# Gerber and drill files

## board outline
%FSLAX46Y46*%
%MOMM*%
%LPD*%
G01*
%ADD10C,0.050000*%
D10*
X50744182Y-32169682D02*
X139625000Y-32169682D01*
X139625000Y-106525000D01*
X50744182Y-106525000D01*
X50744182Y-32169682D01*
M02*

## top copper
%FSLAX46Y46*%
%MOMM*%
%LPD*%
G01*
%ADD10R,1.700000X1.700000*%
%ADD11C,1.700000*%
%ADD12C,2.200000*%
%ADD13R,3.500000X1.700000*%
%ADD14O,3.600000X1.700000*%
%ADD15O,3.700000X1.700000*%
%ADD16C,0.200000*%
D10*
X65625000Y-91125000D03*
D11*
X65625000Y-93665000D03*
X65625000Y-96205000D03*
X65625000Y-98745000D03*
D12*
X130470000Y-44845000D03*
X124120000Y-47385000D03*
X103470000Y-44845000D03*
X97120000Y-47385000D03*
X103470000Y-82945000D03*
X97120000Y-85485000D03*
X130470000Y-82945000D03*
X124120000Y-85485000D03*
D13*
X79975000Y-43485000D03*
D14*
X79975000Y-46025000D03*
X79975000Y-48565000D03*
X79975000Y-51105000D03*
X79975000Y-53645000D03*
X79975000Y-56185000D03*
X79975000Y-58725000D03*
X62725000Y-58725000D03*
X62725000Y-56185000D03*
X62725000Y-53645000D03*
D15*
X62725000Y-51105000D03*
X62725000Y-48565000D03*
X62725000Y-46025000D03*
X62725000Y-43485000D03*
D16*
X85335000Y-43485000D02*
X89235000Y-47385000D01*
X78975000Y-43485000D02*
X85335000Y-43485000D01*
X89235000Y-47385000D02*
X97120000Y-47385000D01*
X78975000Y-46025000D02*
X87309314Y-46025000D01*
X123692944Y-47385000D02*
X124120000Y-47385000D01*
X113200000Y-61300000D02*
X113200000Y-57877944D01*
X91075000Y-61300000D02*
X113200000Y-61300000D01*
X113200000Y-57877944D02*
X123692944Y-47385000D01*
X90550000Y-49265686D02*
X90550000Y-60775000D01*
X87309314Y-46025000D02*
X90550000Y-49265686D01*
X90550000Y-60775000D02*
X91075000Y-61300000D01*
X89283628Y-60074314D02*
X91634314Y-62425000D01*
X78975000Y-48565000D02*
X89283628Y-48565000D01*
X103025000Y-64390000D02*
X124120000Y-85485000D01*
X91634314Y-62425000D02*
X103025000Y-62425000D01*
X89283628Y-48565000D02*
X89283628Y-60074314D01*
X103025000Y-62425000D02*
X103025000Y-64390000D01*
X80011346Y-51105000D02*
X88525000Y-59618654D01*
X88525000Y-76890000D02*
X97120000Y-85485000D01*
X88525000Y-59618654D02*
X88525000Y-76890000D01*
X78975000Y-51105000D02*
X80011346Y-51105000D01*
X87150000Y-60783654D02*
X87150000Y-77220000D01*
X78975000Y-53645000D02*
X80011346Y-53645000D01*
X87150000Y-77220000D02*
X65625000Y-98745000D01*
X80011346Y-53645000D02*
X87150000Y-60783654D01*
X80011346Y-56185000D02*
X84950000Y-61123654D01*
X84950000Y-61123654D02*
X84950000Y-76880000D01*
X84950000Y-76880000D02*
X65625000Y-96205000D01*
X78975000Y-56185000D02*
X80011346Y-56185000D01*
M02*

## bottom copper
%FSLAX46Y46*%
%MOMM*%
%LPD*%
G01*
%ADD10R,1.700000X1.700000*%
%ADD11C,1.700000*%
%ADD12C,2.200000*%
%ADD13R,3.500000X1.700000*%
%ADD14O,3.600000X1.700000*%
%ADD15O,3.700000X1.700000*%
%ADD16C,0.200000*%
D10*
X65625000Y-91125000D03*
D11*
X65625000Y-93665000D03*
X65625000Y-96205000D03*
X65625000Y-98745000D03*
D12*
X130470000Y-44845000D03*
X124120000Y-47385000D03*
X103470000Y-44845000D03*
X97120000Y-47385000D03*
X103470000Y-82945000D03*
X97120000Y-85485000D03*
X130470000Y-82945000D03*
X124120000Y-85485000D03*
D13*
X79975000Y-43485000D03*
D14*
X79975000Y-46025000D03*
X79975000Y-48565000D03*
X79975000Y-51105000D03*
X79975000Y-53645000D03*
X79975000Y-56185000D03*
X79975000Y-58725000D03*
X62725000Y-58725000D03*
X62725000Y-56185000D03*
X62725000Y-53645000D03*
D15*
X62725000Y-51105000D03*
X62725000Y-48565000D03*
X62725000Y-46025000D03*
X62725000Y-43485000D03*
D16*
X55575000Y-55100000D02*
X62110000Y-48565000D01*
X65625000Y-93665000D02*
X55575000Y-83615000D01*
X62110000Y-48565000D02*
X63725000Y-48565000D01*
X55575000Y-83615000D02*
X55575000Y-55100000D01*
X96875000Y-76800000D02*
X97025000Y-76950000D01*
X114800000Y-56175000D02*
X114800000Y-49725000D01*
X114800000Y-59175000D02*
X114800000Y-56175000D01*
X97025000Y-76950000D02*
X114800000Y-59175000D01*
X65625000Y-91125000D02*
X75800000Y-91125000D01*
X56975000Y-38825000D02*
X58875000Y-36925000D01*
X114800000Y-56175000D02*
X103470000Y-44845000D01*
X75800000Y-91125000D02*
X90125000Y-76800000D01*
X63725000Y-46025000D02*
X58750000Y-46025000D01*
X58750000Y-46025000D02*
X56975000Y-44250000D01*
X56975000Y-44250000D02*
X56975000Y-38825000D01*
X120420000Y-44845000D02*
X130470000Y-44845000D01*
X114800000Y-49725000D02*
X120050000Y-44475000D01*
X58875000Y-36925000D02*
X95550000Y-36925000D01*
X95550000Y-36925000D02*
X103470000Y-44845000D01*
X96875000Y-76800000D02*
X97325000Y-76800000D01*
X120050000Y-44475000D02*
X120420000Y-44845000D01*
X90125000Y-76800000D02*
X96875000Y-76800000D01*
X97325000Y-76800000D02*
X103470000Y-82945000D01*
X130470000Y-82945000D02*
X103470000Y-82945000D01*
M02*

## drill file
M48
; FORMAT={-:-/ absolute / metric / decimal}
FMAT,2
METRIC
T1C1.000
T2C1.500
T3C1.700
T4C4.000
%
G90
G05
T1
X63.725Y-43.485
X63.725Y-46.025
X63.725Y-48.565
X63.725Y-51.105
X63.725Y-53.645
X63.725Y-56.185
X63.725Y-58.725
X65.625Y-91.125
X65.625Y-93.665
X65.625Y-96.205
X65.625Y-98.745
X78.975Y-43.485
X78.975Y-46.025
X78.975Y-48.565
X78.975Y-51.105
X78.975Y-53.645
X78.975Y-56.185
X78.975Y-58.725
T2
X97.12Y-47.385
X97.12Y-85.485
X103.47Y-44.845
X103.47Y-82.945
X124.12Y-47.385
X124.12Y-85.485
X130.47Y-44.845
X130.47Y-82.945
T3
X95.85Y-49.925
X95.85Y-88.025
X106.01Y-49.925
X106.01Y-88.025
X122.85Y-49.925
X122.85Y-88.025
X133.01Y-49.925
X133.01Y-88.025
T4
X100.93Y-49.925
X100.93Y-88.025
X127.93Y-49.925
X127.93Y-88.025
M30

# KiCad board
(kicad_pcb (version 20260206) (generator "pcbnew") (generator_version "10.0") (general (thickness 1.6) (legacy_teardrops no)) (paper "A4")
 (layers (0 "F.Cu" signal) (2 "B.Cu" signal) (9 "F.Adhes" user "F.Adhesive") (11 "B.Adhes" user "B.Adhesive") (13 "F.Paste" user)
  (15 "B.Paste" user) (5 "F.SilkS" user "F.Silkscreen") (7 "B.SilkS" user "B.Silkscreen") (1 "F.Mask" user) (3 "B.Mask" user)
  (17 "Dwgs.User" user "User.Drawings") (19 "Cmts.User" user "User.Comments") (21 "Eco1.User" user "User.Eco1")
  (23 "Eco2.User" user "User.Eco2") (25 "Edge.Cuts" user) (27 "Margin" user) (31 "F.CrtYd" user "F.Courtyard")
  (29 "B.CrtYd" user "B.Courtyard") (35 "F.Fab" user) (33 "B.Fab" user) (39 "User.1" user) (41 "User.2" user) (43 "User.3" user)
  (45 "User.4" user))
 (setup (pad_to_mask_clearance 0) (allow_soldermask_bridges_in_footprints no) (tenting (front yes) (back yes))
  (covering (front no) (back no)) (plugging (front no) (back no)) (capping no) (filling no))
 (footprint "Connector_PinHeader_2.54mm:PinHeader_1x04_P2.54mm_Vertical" (layer "F.Cu") (at 65.625 91.125)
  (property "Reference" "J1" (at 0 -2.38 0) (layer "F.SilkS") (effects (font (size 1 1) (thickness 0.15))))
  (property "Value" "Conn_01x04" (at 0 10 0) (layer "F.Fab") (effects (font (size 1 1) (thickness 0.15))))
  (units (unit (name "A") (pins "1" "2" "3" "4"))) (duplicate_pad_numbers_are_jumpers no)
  (pad "1" thru_hole rect (at 0 0) (size 1.7 1.7) (drill 1) (layers "*.Cu" "*.Mask") (remove_unused_layers no) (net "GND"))
  (pad "2" thru_hole circle (at 0 2.54) (size 1.7 1.7) (drill 1) (layers "*.Cu" "*.Mask") (remove_unused_layers no) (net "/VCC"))
  (pad "3" thru_hole circle (at 0 5.08) (size 1.7 1.7) (drill 1) (layers "*.Cu" "*.Mask") (remove_unused_layers no) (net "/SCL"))
  (pad "4" thru_hole circle (at 0 7.62) (size 1.7 1.7) (drill 1) (layers "*.Cu" "*.Mask") (remove_unused_layers no) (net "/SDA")))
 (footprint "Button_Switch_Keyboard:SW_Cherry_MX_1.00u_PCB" (layer "F.Cu") (at 130.47 44.845)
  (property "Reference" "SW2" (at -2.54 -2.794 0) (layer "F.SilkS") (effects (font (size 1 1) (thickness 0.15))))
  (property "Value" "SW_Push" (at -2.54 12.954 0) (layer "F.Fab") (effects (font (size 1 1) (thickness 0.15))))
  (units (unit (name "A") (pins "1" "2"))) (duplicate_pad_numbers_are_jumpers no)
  (pad "" np_thru_hole circle (at -7.62 5.08) (size 1.7 1.7) (drill 1.7) (layers "*.Cu" "*.Mask"))
  (pad "" np_thru_hole circle (at -2.54 5.08) (size 4 4) (drill 4) (layers "*.Cu" "*.Mask"))
  (pad "" np_thru_hole circle (at 2.54 5.08) (size 1.7 1.7) (drill 1.7) (layers "*.Cu" "*.Mask"))
  (pad "1" thru_hole circle (at 0 0) (size 2.2 2.2) (drill 1.5) (layers "*.Cu" "*.Mask") (remove_unused_layers no) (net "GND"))
  (pad "2" thru_hole circle (at -6.35 2.54) (size 2.2 2.2) (drill 1.5) (layers "*.Cu" "*.Mask") (remove_unused_layers no)
   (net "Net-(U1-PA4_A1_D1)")))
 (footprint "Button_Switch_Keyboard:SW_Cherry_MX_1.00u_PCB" (layer "F.Cu") (at 103.47 44.845)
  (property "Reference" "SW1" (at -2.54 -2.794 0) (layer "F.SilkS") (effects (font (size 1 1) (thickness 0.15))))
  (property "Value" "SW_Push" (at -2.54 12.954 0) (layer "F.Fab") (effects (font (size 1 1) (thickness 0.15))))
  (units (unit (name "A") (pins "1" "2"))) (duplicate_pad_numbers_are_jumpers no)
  (pad "" np_thru_hole circle (at -7.62 5.08) (size 1.7 1.7) (drill 1.7) (layers "*.Cu" "*.Mask"))
  (pad "" np_thru_hole circle (at -2.54 5.08) (size 4 4) (drill 4) (layers "*.Cu" "*.Mask"))
  (pad "" np_thru_hole circle (at 2.54 5.08) (size 1.7 1.7) (drill 1.7) (layers "*.Cu" "*.Mask"))
  (pad "1" thru_hole circle (at 0 0) (size 2.2 2.2) (drill 1.5) (layers "*.Cu" "*.Mask") (remove_unused_layers no) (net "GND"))
  (pad "2" thru_hole circle (at -6.35 2.54) (size 2.2 2.2) (drill 1.5) (layers "*.Cu" "*.Mask") (remove_unused_layers no)
   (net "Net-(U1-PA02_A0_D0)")))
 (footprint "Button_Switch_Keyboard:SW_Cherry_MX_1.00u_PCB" (layer "F.Cu") (at 103.47 82.945)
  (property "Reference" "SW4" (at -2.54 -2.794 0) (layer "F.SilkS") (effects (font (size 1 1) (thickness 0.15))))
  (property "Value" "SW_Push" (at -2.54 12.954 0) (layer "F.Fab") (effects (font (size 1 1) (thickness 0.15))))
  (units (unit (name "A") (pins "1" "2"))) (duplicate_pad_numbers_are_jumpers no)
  (pad "" np_thru_hole circle (at -7.62 5.08) (size 1.7 1.7) (drill 1.7) (layers "*.Cu" "*.Mask"))
  (pad "" np_thru_hole circle (at -2.54 5.08) (size 4 4) (drill 4) (layers "*.Cu" "*.Mask"))
  (pad "" np_thru_hole circle (at 2.54 5.08) (size 1.7 1.7) (drill 1.7) (layers "*.Cu" "*.Mask"))
  (pad "1" thru_hole circle (at 0 0) (size 2.2 2.2) (drill 1.5) (layers "*.Cu" "*.Mask") (remove_unused_layers no) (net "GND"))
  (pad "2" thru_hole circle (at -6.35 2.54) (size 2.2 2.2) (drill 1.5) (layers "*.Cu" "*.Mask") (remove_unused_layers no)
   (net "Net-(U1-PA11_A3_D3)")))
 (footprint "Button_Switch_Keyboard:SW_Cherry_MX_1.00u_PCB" (layer "F.Cu") (at 130.47 82.945)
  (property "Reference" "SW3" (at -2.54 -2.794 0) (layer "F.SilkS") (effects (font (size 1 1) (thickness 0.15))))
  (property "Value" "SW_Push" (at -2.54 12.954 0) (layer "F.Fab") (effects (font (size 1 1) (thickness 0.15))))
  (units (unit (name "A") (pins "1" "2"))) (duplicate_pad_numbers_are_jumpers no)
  (pad "" np_thru_hole circle (at -7.62 5.08) (size 1.7 1.7) (drill 1.7) (layers "*.Cu" "*.Mask"))
  (pad "" np_thru_hole circle (at -2.54 5.08) (size 4 4) (drill 4) (layers "*.Cu" "*.Mask"))
  (pad "" np_thru_hole circle (at 2.54 5.08) (size 1.7 1.7) (drill 1.7) (layers "*.Cu" "*.Mask"))
  (pad "1" thru_hole circle (at 0 0) (size 2.2 2.2) (drill 1.5) (layers "*.Cu" "*.Mask") (remove_unused_layers no) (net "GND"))
  (pad "2" thru_hole circle (at -6.35 2.54) (size 2.2 2.2) (drill 1.5) (layers "*.Cu" "*.Mask") (remove_unused_layers no)
   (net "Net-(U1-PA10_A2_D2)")))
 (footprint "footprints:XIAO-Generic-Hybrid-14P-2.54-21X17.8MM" (layer "B.Cu") (at 71.35 51.105 180)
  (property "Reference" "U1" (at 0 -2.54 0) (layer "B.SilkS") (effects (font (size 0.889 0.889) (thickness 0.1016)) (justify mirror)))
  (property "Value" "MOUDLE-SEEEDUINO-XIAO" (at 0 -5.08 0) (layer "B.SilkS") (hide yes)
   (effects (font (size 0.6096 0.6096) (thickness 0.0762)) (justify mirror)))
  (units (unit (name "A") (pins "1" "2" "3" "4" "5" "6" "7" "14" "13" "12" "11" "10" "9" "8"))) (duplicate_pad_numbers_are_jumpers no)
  (pad "1" thru_hole rect (at -7.625 7.62 180) (size 3.5 1.7) (drill 1 (offset -1 0)) (layers "*.Cu" "*.Mask") (remove_unused_layers no)
   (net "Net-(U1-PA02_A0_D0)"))
  (pad "2" thru_hole oval (at -7.625 5.08 180) (size 3.6 1.7) (drill 1 (offset -1 0)) (layers "*.Cu" "*.Mask") (remove_unused_layers no)
   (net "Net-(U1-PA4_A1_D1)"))
  (pad "3" thru_hole oval (at -7.625 2.54 180) (size 3.6 1.7) (drill 1 (offset -1 0)) (layers "*.Cu" "*.Mask") (remove_unused_layers no)
   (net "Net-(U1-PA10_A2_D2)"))
  (pad "4" thru_hole oval (at -7.625 0 180) (size 3.6 1.7) (drill 1 (offset -1 0)) (layers "*.Cu" "*.Mask") (remove_unused_layers no)
   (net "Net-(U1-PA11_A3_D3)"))
  (pad "5" thru_hole oval (at -7.625 -2.54 180) (size 3.6 1.7) (drill 1 (offset -1 0)) (layers "*.Cu" "*.Mask") (remove_unused_layers no)
   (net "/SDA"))
  (pad "6" thru_hole oval (at -7.625 -5.08) (size 3.6 1.7) (drill 1 (offset 1 0)) (layers "*.Cu" "*.Mask") (remove_unused_layers no)
   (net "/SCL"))
  (pad "7" thru_hole oval (at -7.625 -7.62 180) (size 3.6 1.7) (drill 1 (offset -1 0)) (layers "*.Cu" "*.Mask") (remove_unused_layers no)
   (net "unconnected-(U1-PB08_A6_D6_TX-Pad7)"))
  (pad "8" thru_hole oval (at 7.625 -7.62 180) (size 3.6 1.7) (drill 1 (offset 1 0)) (layers "*.Cu" "*.Mask") (remove_unused_layers no)
   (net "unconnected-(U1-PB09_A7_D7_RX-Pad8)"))
  (pad "9" thru_hole oval (at 7.625 -5.08 180) (size 3.6 1.7) (drill 1 (offset 1 0)) (layers "*.Cu" "*.Mask") (remove_unused_layers no)
   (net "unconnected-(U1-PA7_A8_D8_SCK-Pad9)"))
  (pad "10" thru_hole oval (at 7.625 -2.54 180) (size 3.6 1.7) (drill 1 (offset 1 0)) (layers "*.Cu" "*.Mask") (remove_unused_layers no)
   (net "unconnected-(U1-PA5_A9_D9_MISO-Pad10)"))
  (pad "11" thru_hole oval (at 7.625 0 180) (size 3.7 1.7) (drill 1 (offset 1 0)) (layers "*.Cu" "*.Mask") (remove_unused_layers no)
   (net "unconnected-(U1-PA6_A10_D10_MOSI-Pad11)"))
  (pad "12" thru_hole oval (at 7.625 2.54 180) (size 3.7 1.7) (drill 1 (offset 1 0)) (layers "*.Cu" "*.Mask") (remove_unused_layers no)
   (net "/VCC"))
  (pad "13" thru_hole oval (at 7.625 5.08 180) (size 3.7 1.7) (drill 1 (offset 1 0)) (layers "*.Cu" "*.Mask") (remove_unused_layers no)
   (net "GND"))
  (pad "14" thru_hole oval (at 7.625 7.62 180) (size 3.7 1.7) (drill 1 (offset 1 0)) (layers "*.Cu" "*.Mask") (remove_unused_layers no)
   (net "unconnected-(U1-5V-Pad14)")))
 (gr_rect (start 50.744182 32.169682) (end 139.625 106.525) (stroke (width 0.05) (type default)) (fill no) (layer "Edge.Cuts"))
 (segment (start 85.335 43.485) (end 89.235 47.385) (width 0.2) (layer "F.Cu") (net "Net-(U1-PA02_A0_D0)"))
 (segment (start 78.975 43.485) (end 85.335 43.485) (width 0.2) (layer "F.Cu") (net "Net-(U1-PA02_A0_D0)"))
 (segment (start 89.235 47.385) (end 97.12 47.385) (width 0.2) (layer "F.Cu") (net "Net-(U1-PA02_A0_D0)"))
 (segment (start 78.975 46.025) (end 87.309314 46.025) (width 0.2) (layer "F.Cu") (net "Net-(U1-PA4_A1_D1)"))
 (segment (start 123.692944 47.385) (end 124.12 47.385) (width 0.2) (layer "F.Cu") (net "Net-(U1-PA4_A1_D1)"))
 (segment (start 113.2 61.3) (end 113.2 57.877944) (width 0.2) (layer "F.Cu") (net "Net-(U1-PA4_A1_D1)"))
 (segment (start 91.075 61.3) (end 113.2 61.3) (width 0.2) (layer "F.Cu") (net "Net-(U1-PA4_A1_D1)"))
 (segment (start 113.2 57.877944) (end 123.692944 47.385) (width 0.2) (layer "F.Cu") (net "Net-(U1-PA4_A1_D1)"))
 (segment (start 90.55 49.265686) (end 90.55 60.775) (width 0.2) (layer "F.Cu") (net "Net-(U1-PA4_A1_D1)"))
 (segment (start 87.309314 46.025) (end 90.55 49.265686) (width 0.2) (layer "F.Cu") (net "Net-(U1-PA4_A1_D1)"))
 (segment (start 90.55 60.775) (end 91.075 61.3) (width 0.2) (layer "F.Cu") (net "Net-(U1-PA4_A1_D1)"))
 (segment (start 89.283628 60.074314) (end 91.634314 62.425) (width 0.2) (layer "F.Cu") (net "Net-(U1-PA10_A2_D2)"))
 (segment (start 78.975 48.565) (end 89.283628 48.565) (width 0.2) (layer "F.Cu") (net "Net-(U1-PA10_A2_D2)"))
 (segment (start 103.025 64.39) (end 124.12 85.485) (width 0.2) (layer "F.Cu") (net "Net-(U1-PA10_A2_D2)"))
 (segment (start 91.634314 62.425) (end 103.025 62.425) (width 0.2) (layer "F.Cu") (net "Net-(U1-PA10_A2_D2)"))
 (segment (start 89.283628 48.565) (end 89.283628 60.074314) (width 0.2) (layer "F.Cu") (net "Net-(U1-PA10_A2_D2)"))
 (segment (start 103.025 62.425) (end 103.025 64.39) (width 0.2) (layer "F.Cu") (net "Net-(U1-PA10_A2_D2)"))
 (segment (start 80.011346 51.105) (end 88.525 59.618654) (width 0.2) (layer "F.Cu") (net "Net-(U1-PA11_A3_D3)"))
 (segment (start 88.525 76.89) (end 97.12 85.485) (width 0.2) (layer "F.Cu") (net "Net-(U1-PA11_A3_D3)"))
 (segment (start 88.525 59.618654) (end 88.525 76.89) (width 0.2) (layer "F.Cu") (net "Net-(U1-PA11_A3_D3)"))
 (segment (start 78.975 51.105) (end 80.011346 51.105) (width 0.2) (layer "F.Cu") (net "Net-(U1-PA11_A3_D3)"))
 (segment (start 87.15 60.783654) (end 87.15 77.22) (width 0.2) (layer "F.Cu") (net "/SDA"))
 (segment (start 78.975 53.645) (end 80.011346 53.645) (width 0.2) (layer "F.Cu") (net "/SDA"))
 (segment (start 87.15 77.22) (end 65.625 98.745) (width 0.2) (layer "F.Cu") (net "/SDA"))
 (segment (start 80.011346 53.645) (end 87.15 60.783654) (width 0.2) (layer "F.Cu") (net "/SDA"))
 (segment (start 80.011346 56.185) (end 84.95 61.123654) (width 0.2) (layer "F.Cu") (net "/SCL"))
 (segment (start 84.95 61.123654) (end 84.95 76.88) (width 0.2) (layer "F.Cu") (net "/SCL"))
 (segment (start 84.95 76.88) (end 65.625 96.205) (width 0.2) (layer "F.Cu") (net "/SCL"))
 (segment (start 78.975 56.185) (end 80.011346 56.185) (width 0.2) (layer "F.Cu") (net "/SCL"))
 (segment (start 55.575 55.1) (end 62.11 48.565) (width 0.2) (layer "B.Cu") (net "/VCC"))
 (segment (start 65.625 93.665) (end 55.575 83.615) (width 0.2) (layer "B.Cu") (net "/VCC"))
 (segment (start 62.11 48.565) (end 63.725 48.565) (width 0.2) (layer "B.Cu") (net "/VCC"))
 (segment (start 55.575 83.615) (end 55.575 55.1) (width 0.2) (layer "B.Cu") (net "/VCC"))
 (segment (start 96.875 76.8) (end 97.025 76.95) (width 0.2) (layer "B.Cu") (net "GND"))
 (segment (start 114.8 56.175) (end 114.8 49.725) (width 0.2) (layer "B.Cu") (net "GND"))
 (segment (start 114.8 59.175) (end 114.8 56.175) (width 0.2) (layer "B.Cu") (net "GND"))
 (segment (start 97.025 76.95) (end 114.8 59.175) (width 0.2) (layer "B.Cu") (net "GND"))
 (segment (start 65.625 91.125) (end 75.8 91.125) (width 0.2) (layer "B.Cu") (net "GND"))
 (segment (start 56.975 38.825) (end 58.875 36.925) (width 0.2) (layer "B.Cu") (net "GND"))
 (segment (start 114.8 56.175) (end 103.47 44.845) (width 0.2) (layer "B.Cu") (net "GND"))
 (segment (start 75.8 91.125) (end 90.125 76.8) (width 0.2) (layer "B.Cu") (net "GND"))
 (segment (start 63.725 46.025) (end 58.75 46.025) (width 0.2) (layer "B.Cu") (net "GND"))
 (segment (start 58.75 46.025) (end 56.975 44.25) (width 0.2) (layer "B.Cu") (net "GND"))
 (segment (start 56.975 44.25) (end 56.975 38.825) (width 0.2) (layer "B.Cu") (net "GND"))
 (segment (start 120.42 44.845) (end 130.47 44.845) (width 0.2) (layer "B.Cu") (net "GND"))
 (segment (start 114.8 49.725) (end 120.05 44.475) (width 0.2) (layer "B.Cu") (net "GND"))
 (segment (start 58.875 36.925) (end 95.55 36.925) (width 0.2) (layer "B.Cu") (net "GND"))
 (segment (start 95.55 36.925) (end 103.47 44.845) (width 0.2) (layer "B.Cu") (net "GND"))
 (segment (start 96.875 76.8) (end 97.325 76.8) (width 0.2) (layer "B.Cu") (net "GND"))
 (segment (start 120.05 44.475) (end 120.42 44.845) (width 0.2) (layer "B.Cu") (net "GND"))
 (segment (start 90.125 76.8) (end 96.875 76.8) (width 0.2) (layer "B.Cu") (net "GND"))
 (segment (start 97.325 76.8) (end 103.47 82.945) (width 0.2) (layer "B.Cu") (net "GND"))
 (segment (start 130.47 82.945) (end 103.47 82.945) (width 0.2) (layer "B.Cu") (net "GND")))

